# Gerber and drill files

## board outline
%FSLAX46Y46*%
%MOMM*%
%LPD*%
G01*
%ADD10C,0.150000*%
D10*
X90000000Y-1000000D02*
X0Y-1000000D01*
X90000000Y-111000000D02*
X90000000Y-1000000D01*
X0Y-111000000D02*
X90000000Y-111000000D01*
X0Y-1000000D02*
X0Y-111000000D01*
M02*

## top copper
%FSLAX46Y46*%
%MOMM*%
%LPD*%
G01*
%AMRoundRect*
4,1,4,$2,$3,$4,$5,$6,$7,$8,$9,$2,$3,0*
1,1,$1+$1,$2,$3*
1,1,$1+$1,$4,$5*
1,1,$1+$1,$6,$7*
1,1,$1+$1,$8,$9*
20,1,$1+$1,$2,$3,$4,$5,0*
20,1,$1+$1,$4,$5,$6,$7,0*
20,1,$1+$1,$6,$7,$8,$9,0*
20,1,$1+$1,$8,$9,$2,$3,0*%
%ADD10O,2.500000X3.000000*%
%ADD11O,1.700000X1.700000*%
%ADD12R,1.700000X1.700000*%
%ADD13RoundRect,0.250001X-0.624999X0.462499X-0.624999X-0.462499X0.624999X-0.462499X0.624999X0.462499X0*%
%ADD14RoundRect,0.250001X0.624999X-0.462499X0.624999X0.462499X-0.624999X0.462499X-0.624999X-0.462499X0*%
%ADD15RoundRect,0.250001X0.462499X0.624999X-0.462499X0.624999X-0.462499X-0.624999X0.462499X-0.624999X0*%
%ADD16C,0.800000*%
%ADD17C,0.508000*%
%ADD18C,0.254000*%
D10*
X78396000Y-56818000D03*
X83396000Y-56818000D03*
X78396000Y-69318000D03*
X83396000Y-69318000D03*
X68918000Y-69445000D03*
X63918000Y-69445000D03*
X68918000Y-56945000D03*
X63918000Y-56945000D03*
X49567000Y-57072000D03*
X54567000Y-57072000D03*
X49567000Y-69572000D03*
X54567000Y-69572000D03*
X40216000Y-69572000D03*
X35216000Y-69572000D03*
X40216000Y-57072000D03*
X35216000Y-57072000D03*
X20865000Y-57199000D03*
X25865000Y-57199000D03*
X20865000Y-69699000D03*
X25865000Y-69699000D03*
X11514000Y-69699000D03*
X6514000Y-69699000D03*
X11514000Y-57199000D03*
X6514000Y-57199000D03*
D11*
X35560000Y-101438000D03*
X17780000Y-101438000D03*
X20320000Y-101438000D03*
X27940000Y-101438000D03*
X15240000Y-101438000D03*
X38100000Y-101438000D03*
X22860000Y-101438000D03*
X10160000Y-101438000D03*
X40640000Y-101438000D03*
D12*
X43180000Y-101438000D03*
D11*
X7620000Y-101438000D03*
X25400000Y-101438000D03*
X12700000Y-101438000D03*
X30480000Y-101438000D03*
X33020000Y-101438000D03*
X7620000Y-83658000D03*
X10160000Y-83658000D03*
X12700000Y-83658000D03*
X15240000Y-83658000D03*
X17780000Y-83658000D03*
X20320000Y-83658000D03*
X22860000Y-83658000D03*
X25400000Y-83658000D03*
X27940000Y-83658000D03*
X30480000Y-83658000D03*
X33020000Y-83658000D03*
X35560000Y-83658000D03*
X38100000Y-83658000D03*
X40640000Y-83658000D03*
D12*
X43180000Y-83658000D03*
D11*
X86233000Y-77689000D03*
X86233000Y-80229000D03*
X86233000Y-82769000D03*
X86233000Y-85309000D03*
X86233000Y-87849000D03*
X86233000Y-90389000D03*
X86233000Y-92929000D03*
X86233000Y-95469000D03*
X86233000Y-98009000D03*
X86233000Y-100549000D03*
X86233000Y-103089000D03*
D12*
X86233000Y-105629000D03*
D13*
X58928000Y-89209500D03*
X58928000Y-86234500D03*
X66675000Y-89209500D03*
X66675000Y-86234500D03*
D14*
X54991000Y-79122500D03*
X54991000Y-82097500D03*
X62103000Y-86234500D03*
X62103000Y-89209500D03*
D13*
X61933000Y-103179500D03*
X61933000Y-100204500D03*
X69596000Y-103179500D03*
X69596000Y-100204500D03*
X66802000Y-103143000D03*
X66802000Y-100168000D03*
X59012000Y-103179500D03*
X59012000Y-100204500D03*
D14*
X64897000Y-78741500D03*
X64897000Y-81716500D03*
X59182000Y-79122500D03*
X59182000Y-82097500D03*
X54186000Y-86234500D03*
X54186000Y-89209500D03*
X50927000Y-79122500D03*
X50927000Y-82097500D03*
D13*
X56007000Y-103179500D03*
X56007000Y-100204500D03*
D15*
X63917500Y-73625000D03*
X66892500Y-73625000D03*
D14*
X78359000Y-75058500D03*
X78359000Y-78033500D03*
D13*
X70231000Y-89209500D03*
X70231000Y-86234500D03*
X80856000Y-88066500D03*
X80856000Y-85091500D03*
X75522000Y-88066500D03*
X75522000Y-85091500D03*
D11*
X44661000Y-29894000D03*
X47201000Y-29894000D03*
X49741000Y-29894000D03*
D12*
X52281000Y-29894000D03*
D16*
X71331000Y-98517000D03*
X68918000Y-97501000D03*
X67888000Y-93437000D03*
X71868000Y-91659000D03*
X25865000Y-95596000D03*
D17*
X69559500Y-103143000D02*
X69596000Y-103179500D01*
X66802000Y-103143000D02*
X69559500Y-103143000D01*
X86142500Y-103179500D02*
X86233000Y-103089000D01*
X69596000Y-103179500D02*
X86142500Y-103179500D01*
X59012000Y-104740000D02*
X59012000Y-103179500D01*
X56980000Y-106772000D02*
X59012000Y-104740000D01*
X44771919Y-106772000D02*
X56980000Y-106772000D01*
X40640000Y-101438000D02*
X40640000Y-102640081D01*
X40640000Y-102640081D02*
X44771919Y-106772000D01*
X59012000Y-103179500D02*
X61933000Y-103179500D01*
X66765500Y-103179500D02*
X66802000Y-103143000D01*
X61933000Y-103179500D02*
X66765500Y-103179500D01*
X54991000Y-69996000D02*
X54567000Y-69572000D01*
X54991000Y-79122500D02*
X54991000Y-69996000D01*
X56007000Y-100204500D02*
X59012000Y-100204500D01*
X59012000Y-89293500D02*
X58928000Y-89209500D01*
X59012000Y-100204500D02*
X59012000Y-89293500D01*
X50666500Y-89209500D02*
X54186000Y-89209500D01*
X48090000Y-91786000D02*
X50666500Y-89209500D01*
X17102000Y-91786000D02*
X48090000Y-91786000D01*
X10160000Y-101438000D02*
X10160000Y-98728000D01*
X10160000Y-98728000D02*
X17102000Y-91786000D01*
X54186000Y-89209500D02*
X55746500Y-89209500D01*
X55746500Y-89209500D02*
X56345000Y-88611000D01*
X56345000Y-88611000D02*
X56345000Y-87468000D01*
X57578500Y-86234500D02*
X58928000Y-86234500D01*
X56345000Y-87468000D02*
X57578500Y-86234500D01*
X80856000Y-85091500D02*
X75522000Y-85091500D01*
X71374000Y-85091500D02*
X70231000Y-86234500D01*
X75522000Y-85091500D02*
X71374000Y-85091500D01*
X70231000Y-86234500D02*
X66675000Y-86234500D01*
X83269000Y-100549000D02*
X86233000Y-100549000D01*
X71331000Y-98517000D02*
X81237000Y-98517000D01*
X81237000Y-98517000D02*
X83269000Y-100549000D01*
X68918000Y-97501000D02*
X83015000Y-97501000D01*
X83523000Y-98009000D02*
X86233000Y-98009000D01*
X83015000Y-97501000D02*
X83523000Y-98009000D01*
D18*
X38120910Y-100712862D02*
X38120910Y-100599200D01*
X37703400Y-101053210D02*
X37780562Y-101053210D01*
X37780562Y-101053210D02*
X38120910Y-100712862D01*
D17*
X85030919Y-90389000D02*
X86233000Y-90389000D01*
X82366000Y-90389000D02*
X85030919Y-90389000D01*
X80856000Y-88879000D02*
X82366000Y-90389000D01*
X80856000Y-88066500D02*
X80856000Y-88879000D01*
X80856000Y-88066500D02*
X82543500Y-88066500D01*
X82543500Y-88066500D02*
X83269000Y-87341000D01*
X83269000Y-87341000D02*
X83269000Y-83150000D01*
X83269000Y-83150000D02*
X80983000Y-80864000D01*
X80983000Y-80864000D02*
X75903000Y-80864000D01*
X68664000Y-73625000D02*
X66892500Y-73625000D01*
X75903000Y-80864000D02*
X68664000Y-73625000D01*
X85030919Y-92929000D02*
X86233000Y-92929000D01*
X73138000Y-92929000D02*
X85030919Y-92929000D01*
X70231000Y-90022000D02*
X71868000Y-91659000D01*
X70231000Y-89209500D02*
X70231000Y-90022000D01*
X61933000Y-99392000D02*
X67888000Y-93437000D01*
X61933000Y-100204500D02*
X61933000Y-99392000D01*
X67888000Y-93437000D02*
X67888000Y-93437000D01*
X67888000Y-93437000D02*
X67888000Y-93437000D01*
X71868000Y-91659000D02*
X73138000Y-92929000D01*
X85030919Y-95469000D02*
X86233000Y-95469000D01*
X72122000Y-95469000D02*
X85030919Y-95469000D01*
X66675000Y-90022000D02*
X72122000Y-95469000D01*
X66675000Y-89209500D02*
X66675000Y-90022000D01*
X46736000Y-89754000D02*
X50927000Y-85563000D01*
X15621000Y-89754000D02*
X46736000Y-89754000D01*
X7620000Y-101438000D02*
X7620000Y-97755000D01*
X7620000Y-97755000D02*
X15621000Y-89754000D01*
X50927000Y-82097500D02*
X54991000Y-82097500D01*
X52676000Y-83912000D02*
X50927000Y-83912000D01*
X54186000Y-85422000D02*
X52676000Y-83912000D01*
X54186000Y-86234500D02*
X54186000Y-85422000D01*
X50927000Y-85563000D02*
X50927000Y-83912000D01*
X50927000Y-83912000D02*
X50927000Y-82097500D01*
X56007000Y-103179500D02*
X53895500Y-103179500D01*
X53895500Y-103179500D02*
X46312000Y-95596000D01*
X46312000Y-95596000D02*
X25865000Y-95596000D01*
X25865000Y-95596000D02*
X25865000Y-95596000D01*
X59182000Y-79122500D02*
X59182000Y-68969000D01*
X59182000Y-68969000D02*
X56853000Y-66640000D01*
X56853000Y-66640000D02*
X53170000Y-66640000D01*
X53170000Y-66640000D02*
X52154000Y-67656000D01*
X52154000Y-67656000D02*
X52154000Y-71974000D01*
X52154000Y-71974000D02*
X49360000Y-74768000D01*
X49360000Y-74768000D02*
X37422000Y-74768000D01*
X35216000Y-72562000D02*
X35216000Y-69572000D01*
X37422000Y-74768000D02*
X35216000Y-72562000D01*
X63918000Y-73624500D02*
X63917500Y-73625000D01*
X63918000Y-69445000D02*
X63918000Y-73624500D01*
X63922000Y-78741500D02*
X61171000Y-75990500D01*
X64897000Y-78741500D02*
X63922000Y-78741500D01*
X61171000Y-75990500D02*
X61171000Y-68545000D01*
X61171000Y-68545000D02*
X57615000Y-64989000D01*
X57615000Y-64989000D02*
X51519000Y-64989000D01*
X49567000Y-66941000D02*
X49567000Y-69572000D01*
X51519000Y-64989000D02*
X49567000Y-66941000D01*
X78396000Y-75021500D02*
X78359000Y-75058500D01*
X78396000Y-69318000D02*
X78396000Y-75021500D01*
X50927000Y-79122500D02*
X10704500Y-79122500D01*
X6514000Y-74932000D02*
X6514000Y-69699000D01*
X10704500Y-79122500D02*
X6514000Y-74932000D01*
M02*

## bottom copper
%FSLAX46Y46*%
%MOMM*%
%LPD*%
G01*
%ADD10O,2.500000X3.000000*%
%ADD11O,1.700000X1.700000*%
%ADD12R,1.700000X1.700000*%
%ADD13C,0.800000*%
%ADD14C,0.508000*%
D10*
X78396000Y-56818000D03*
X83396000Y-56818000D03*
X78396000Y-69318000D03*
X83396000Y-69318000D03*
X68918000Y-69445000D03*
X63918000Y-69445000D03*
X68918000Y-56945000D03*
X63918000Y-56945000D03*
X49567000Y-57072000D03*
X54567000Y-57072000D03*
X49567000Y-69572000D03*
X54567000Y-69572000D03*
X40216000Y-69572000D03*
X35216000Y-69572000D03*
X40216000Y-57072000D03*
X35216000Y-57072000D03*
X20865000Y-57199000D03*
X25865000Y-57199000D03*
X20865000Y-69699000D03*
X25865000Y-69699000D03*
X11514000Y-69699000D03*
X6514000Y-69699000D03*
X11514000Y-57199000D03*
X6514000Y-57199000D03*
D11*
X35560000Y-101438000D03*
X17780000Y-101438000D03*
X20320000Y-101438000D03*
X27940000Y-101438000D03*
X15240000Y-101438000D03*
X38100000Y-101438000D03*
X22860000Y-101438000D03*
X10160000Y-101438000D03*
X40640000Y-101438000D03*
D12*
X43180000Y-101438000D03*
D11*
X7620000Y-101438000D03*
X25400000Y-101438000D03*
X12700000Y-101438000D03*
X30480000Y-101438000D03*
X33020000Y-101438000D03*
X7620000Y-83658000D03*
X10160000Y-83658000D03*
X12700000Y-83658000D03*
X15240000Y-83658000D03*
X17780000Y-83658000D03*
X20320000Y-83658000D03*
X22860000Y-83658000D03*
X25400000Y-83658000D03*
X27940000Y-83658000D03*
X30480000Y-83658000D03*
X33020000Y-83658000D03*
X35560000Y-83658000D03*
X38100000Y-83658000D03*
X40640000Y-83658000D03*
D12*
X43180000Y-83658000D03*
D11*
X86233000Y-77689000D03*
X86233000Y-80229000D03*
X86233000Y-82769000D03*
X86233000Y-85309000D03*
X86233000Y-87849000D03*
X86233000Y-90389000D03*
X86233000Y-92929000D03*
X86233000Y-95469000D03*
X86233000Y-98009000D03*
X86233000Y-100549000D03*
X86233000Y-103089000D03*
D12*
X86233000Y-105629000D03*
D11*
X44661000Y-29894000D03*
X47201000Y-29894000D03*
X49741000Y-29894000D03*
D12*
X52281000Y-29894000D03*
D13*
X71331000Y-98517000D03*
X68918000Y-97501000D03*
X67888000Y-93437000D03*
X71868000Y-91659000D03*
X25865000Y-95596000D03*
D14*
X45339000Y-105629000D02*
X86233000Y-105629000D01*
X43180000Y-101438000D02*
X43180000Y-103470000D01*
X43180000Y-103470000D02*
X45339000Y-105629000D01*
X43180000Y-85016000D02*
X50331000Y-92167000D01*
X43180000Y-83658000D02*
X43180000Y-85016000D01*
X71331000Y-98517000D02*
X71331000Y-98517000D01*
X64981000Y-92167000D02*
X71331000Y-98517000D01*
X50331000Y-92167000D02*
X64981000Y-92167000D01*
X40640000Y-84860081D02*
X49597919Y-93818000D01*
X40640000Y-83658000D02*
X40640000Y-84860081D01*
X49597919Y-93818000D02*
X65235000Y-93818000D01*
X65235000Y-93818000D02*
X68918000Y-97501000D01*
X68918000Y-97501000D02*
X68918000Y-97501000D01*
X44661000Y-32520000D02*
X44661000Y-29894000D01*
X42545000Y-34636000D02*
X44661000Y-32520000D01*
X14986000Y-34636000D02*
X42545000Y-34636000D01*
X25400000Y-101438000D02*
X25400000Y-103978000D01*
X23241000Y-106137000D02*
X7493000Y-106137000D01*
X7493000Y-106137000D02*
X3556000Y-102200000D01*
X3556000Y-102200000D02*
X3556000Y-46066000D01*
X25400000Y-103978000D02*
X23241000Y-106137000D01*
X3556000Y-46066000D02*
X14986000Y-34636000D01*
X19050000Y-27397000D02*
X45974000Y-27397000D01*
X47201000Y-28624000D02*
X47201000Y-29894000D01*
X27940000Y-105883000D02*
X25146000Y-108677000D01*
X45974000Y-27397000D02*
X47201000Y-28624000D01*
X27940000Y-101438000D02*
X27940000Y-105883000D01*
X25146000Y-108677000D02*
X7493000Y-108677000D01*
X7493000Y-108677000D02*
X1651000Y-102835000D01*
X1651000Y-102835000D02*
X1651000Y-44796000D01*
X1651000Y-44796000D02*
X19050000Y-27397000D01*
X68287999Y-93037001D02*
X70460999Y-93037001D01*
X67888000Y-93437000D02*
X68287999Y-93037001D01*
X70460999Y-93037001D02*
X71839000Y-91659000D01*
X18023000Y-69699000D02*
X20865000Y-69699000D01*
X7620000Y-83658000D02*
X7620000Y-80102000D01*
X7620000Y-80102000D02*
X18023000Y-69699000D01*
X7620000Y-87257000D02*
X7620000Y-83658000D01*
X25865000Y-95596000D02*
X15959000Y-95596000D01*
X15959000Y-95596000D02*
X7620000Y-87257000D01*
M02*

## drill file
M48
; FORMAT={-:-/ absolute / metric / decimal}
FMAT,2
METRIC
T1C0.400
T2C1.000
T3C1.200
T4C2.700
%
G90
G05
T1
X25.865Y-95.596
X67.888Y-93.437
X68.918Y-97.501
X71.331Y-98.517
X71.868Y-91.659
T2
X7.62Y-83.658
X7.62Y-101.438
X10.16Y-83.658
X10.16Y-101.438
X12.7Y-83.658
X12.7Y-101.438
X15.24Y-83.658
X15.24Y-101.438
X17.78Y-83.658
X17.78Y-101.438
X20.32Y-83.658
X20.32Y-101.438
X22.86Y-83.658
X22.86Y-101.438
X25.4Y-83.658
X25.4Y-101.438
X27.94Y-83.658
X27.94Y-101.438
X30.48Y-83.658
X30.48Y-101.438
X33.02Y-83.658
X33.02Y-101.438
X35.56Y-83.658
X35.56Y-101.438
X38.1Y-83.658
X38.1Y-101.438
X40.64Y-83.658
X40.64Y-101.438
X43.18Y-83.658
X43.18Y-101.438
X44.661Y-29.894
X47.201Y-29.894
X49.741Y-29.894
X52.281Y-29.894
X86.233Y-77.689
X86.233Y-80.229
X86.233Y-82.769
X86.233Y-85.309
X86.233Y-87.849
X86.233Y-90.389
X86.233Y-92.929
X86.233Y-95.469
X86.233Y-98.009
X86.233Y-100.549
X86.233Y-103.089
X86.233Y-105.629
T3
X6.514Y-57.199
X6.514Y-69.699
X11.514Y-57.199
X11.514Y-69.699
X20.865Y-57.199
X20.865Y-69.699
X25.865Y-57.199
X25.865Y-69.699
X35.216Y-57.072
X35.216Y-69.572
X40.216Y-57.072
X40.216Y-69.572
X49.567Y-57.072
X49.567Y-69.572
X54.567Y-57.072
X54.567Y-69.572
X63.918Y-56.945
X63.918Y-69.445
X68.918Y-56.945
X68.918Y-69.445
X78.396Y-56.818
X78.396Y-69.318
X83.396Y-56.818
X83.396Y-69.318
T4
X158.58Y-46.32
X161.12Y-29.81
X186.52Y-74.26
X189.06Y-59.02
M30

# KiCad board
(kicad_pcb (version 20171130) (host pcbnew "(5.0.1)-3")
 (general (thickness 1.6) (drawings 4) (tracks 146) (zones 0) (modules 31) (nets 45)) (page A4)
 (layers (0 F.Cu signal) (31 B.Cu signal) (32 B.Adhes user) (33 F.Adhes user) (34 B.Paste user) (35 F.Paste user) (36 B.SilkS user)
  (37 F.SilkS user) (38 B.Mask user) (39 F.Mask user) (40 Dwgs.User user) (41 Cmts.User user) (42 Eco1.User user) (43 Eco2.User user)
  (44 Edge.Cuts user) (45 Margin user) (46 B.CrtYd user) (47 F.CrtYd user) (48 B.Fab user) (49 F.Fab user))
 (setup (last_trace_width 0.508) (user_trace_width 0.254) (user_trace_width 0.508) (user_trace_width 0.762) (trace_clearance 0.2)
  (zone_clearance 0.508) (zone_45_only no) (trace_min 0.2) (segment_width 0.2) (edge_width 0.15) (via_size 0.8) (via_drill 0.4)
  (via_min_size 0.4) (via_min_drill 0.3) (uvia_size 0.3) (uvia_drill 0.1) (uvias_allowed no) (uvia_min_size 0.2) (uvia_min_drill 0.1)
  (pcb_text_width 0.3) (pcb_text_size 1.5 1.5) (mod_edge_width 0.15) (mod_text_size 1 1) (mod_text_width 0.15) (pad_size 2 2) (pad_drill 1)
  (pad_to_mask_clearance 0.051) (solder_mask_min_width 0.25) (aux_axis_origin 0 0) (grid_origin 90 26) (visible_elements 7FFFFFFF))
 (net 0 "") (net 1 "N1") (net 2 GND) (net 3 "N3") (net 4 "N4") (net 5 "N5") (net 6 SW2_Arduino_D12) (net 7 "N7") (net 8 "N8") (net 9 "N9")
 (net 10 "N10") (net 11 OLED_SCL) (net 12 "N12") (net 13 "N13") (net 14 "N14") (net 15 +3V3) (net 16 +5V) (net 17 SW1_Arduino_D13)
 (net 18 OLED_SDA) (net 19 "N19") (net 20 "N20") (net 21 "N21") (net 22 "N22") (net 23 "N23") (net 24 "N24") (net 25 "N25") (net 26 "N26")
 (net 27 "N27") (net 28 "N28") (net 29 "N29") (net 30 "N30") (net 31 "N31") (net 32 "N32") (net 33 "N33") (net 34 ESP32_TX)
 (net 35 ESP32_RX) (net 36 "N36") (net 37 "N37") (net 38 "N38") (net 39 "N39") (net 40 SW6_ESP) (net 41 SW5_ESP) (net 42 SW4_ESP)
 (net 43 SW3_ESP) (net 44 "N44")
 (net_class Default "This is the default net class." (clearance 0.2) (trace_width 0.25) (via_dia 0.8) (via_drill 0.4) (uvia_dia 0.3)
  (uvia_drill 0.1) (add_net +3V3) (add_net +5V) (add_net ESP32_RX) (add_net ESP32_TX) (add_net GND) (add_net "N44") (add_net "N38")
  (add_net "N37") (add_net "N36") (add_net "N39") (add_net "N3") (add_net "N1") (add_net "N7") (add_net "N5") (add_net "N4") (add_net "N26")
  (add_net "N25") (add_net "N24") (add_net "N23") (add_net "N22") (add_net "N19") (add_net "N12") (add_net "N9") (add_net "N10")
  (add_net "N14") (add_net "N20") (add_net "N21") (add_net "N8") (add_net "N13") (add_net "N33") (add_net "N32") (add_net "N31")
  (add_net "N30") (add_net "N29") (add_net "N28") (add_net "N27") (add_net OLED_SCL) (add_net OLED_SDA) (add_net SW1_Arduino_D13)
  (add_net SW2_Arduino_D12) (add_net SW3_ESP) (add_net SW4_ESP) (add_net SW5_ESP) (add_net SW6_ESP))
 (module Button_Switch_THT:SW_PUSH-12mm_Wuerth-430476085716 (layer F.Cu) (at 83.396 56.818 270)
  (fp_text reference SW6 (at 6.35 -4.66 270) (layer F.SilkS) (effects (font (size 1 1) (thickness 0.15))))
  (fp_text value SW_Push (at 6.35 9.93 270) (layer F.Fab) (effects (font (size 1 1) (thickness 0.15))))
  (pad 2 thru_hole oval (at 0 5 270) (size 3 2.5) (drill 1.2) (layers *.Cu *.Mask) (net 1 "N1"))
  (pad 1 thru_hole oval (at 0 0 270) (size 3 2.5) (drill 1.2) (layers *.Cu *.Mask) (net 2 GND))
  (pad 2 thru_hole oval (at 12.5 5 270) (size 3 2.5) (drill 1.2) (layers *.Cu *.Mask) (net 1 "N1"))
  (pad 1 thru_hole oval (at 12.5 0 270) (size 3 2.5) (drill 1.2) (layers *.Cu *.Mask) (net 2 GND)))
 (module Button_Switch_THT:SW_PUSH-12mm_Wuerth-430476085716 (layer F.Cu) (at 68.918 56.945 270)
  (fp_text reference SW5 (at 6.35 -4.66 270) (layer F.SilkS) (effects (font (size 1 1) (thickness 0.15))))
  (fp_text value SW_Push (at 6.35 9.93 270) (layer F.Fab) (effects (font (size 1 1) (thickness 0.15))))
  (pad 1 thru_hole oval (at 12.5 0 270) (size 3 2.5) (drill 1.2) (layers *.Cu *.Mask) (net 2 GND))
  (pad 2 thru_hole oval (at 12.5 5 270) (size 3 2.5) (drill 1.2) (layers *.Cu *.Mask) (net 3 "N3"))
  (pad 1 thru_hole oval (at 0 0 270) (size 3 2.5) (drill 1.2) (layers *.Cu *.Mask) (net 2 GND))
  (pad 2 thru_hole oval (at 0 5 270) (size 3 2.5) (drill 1.2) (layers *.Cu *.Mask) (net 3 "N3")))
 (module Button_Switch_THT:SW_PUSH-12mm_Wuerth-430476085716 (layer F.Cu) (at 54.567 57.072 270)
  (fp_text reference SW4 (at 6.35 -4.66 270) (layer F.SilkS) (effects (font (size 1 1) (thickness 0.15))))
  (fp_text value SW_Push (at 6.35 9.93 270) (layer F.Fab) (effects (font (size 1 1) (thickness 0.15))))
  (pad 2 thru_hole oval (at 0 5 270) (size 3 2.5) (drill 1.2) (layers *.Cu *.Mask) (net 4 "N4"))
  (pad 1 thru_hole oval (at 0 0 270) (size 3 2.5) (drill 1.2) (layers *.Cu *.Mask) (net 2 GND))
  (pad 2 thru_hole oval (at 12.5 5 270) (size 3 2.5) (drill 1.2) (layers *.Cu *.Mask) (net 4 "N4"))
  (pad 1 thru_hole oval (at 12.5 0 270) (size 3 2.5) (drill 1.2) (layers *.Cu *.Mask) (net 2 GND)))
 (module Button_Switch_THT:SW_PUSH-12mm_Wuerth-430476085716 (layer F.Cu) (at 40.216 57.072 270)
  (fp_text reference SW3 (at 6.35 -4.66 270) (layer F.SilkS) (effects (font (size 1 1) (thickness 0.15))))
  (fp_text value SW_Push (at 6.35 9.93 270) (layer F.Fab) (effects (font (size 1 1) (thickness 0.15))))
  (pad 1 thru_hole oval (at 12.5 0 270) (size 3 2.5) (drill 1.2) (layers *.Cu *.Mask) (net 2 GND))
  (pad 2 thru_hole oval (at 12.5 5 270) (size 3 2.5) (drill 1.2) (layers *.Cu *.Mask) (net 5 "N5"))
  (pad 1 thru_hole oval (at 0 0 270) (size 3 2.5) (drill 1.2) (layers *.Cu *.Mask) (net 2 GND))
  (pad 2 thru_hole oval (at 0 5 270) (size 3 2.5) (drill 1.2) (layers *.Cu *.Mask) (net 5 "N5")))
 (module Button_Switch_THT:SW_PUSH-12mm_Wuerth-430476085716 (layer F.Cu) (at 25.865 57.199 270)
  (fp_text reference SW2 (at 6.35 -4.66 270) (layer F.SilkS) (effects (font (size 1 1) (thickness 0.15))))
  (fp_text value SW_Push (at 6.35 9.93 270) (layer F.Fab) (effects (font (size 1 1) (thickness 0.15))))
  (pad 2 thru_hole oval (at 0 5 270) (size 3 2.5) (drill 1.2) (layers *.Cu *.Mask) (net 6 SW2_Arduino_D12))
  (pad 1 thru_hole oval (at 0 0 270) (size 3 2.5) (drill 1.2) (layers *.Cu *.Mask) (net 2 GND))
  (pad 2 thru_hole oval (at 12.5 5 270) (size 3 2.5) (drill 1.2) (layers *.Cu *.Mask) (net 6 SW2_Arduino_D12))
  (pad 1 thru_hole oval (at 12.5 0 270) (size 3 2.5) (drill 1.2) (layers *.Cu *.Mask) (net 2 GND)))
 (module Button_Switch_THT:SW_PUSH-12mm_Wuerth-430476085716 (layer F.Cu) (at 11.514 57.199 270)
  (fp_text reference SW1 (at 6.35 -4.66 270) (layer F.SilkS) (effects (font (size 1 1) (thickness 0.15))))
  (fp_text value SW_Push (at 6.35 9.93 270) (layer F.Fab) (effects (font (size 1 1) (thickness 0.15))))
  (pad 1 thru_hole oval (at 12.5 0 270) (size 3 2.5) (drill 1.2) (layers *.Cu *.Mask) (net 2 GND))
  (pad 2 thru_hole oval (at 12.5 5 270) (size 3 2.5) (drill 1.2) (layers *.Cu *.Mask) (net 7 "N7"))
  (pad 1 thru_hole oval (at 0 0 270) (size 3 2.5) (drill 1.2) (layers *.Cu *.Mask) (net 2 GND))
  (pad 2 thru_hole oval (at 0 5 270) (size 3 2.5) (drill 1.2) (layers *.Cu *.Mask) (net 7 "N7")))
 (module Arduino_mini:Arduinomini (layer F.Cu) (at 43.18 91.278 270)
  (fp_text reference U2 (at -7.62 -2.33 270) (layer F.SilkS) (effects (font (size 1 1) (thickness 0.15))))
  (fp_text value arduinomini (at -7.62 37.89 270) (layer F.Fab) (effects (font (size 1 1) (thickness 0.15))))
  (pad 27 thru_hole oval (at 10.16 7.62 270) (size 1.7 1.7) (drill 1) (layers *.Cu *.Mask) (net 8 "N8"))
  (pad 20 thru_hole oval (at 10.16 25.4 270) (size 1.7 1.7) (drill 1) (layers *.Cu *.Mask) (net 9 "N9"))
  (pad 21 thru_hole oval (at 10.16 22.86 270) (size 1.7 1.7) (drill 1) (layers *.Cu *.Mask) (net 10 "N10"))
  (pad 24 thru_hole oval (at 10.16 15.24 270) (size 1.7 1.7) (drill 1) (layers *.Cu *.Mask) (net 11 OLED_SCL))
  (pad 19 thru_hole oval (at 10.16 27.94 270) (size 1.7 1.7) (drill 1) (layers *.Cu *.Mask) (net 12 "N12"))
  (pad 28 thru_hole oval (at 10.16 5.08 270) (size 1.7 1.7) (drill 1) (layers *.Cu *.Mask) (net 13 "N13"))
  (pad 22 thru_hole oval (at 10.16 20.32 270) (size 1.7 1.7) (drill 1) (layers *.Cu *.Mask) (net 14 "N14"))
  (pad 17 thru_hole oval (at 10.16 33.02 270) (size 1.7 1.7) (drill 1) (layers *.Cu *.Mask) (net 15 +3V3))
  (pad 29 thru_hole oval (at 10.16 2.54 270) (size 1.7 1.7) (drill 1) (layers *.Cu *.Mask) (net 2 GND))
  (pad 30 thru_hole rect (at 10.16 0 270) (size 1.7 1.7) (drill 1) (layers *.Cu *.Mask) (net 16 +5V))
  (pad 16 thru_hole oval (at 10.16 35.56 270) (size 1.7 1.7) (drill 1) (layers *.Cu *.Mask) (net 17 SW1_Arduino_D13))
  (pad 23 thru_hole oval (at 10.16 17.78 270) (size 1.7 1.7) (drill 1) (layers *.Cu *.Mask) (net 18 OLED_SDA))
  (pad 18 thru_hole oval (at 10.16 30.48 270) (size 1.7 1.7) (drill 1) (layers *.Cu *.Mask) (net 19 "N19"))
  (pad 25 thru_hole oval (at 10.16 12.7 270) (size 1.7 1.7) (drill 1) (layers *.Cu *.Mask) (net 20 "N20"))
  (pad 26 thru_hole oval (at 10.16 10.16 270) (size 1.7 1.7) (drill 1) (layers *.Cu *.Mask) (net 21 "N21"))
  (pad 15 thru_hole oval (at -7.62 35.56 270) (size 1.7 1.7) (drill 1) (layers *.Cu *.Mask) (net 6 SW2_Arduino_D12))
  (pad 14 thru_hole oval (at -7.62 33.02 270) (size 1.7 1.7) (drill 1) (layers *.Cu *.Mask) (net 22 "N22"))
  (pad 13 thru_hole oval (at -7.62 30.48 270) (size 1.7 1.7) (drill 1) (layers *.Cu *.Mask) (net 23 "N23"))
  (pad 12 thru_hole oval (at -7.62 27.94 270) (size 1.7 1.7) (drill 1) (layers *.Cu *.Mask) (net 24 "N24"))
  (pad 11 thru_hole oval (at -7.62 25.4 270) (size 1.7 1.7) (drill 1) (layers *.Cu *.Mask) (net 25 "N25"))
  (pad 10 thru_hole oval (at -7.62 22.86 270) (size 1.7 1.7) (drill 1) (layers *.Cu *.Mask) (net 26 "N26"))
  (pad 9 thru_hole oval (at -7.62 20.32 270) (size 1.7 1.7) (drill 1) (layers *.Cu *.Mask) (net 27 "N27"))
  (pad 8 thru_hole oval (at -7.62 17.78 270) (size 1.7 1.7) (drill 1) (layers *.Cu *.Mask) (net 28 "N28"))
  (pad 7 thru_hole oval (at -7.62 15.24 270) (size 1.7 1.7) (drill 1) (layers *.Cu *.Mask) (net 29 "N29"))
  (pad 6 thru_hole oval (at -7.62 12.7 270) (size 1.7 1.7) (drill 1) (layers *.Cu *.Mask) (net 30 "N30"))
  (pad 5 thru_hole oval (at -7.62 10.16 270) (size 1.7 1.7) (drill 1) (layers *.Cu *.Mask) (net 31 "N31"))
  (pad 4 thru_hole oval (at -7.62 7.62 270) (size 1.7 1.7) (drill 1) (layers *.Cu *.Mask) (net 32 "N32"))
  (pad 3 thru_hole oval (at -7.62 5.08 270) (size 1.7 1.7) (drill 1) (layers *.Cu *.Mask) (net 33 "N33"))
  (pad 2 thru_hole oval (at -7.62 2.54 270) (size 1.7 1.7) (drill 1) (layers *.Cu *.Mask) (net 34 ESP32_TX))
  (pad 1 thru_hole rect (at -7.62 0 270) (size 1.7 1.7) (drill 1) (layers *.Cu *.Mask) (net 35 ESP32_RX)))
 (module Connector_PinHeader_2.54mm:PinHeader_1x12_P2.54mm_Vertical (layer F.Cu) (at 86.233 105.629 180)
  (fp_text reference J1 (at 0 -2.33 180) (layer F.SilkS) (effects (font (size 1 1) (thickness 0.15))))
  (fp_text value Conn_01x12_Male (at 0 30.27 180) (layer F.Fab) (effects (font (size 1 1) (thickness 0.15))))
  (pad 12 thru_hole oval (at 0 27.94 180) (size 1.7 1.7) (drill 1) (layers *.Cu *.Mask) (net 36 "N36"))
  (pad 11 thru_hole oval (at 0 25.4 180) (size 1.7 1.7) (drill 1) (layers *.Cu *.Mask) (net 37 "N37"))
  (pad 10 thru_hole oval (at 0 22.86 180) (size 1.7 1.7) (drill 1) (layers *.Cu *.Mask) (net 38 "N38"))
  (pad 9 thru_hole oval (at 0 20.32 180) (size 1.7 1.7) (drill 1) (layers *.Cu *.Mask) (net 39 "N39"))
  (pad 8 thru_hole oval (at 0 17.78 180) (size 1.7 1.7) (drill 1) (layers *.Cu *.Mask) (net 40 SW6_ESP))
  (pad 7 thru_hole oval (at 0 15.24 180) (size 1.7 1.7) (drill 1) (layers *.Cu *.Mask) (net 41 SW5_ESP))
  (pad 6 thru_hole oval (at 0 12.7 180) (size 1.7 1.7) (drill 1) (layers *.Cu *.Mask) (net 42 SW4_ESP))
  (pad 5 thru_hole oval (at 0 10.16 180) (size 1.7 1.7) (drill 1) (layers *.Cu *.Mask) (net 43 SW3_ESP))
  (pad 4 thru_hole oval (at 0 7.62 180) (size 1.7 1.7) (drill 1) (layers *.Cu *.Mask) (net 34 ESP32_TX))
  (pad 3 thru_hole oval (at 0 5.08 180) (size 1.7 1.7) (drill 1) (layers *.Cu *.Mask) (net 35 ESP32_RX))
  (pad 2 thru_hole oval (at 0 2.54 180) (size 1.7 1.7) (drill 1) (layers *.Cu *.Mask) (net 2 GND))
  (pad 1 thru_hole rect (at 0 0 180) (size 1.7 1.7) (drill 1) (layers *.Cu *.Mask) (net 16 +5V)))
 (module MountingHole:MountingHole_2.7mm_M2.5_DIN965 (layer F.Cu) (at 186.52 74.26)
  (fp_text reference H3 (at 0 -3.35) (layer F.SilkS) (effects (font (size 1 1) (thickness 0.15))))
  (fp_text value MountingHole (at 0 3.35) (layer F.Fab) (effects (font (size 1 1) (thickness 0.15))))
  (pad 1 np_thru_hole circle (at 0 0) (size 2.7 2.7) (drill 2.7) (layers *.Cu *.Mask)))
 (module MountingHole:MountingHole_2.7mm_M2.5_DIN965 (layer F.Cu) (at 158.58 46.32)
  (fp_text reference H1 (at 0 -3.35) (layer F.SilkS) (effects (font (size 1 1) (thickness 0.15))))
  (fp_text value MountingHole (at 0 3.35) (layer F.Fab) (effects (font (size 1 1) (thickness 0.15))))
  (pad 1 np_thru_hole circle (at 0 0) (size 2.7 2.7) (drill 2.7) (layers *.Cu *.Mask)))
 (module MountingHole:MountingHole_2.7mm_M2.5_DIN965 (layer F.Cu) (at 189.06 59.02)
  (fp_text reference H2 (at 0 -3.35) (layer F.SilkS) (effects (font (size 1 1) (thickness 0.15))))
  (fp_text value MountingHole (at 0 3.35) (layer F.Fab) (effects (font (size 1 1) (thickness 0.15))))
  (pad 1 np_thru_hole circle (at 0 0) (size 2.7 2.7) (drill 2.7) (layers *.Cu *.Mask)))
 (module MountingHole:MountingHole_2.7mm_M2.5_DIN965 (layer F.Cu) (at 161.12 29.81)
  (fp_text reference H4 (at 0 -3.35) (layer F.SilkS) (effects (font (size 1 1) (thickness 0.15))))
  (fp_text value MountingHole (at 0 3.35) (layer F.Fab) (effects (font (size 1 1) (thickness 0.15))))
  (pad 1 np_thru_hole circle (at 0 0) (size 2.7 2.7) (drill 2.7) (layers *.Cu *.Mask)))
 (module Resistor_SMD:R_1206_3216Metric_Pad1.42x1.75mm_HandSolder (layer F.Cu) (at 58.928 87.722 270)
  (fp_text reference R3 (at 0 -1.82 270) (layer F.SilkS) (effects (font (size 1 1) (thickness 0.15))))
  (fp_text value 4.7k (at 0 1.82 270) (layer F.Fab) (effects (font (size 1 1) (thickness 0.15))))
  (pad 2 smd roundrect (at 1.4875 0 270) (size 1.425 1.75) (layers F.Cu F.Paste F.Mask) (roundrect_rratio 0.175439) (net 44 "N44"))
  (pad 1 smd roundrect (at -1.4875 0 270) (size 1.425 1.75) (layers F.Cu F.Paste F.Mask) (roundrect_rratio 0.175439) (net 15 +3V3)))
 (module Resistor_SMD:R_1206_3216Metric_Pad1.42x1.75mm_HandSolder (layer F.Cu) (at 66.675 87.722 270)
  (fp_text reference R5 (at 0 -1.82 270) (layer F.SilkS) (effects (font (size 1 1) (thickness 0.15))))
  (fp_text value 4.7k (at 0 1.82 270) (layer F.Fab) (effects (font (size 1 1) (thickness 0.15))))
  (pad 2 smd roundrect (at 1.4875 0 270) (size 1.425 1.75) (layers F.Cu F.Paste F.Mask) (roundrect_rratio 0.175439) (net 43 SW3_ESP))
  (pad 1 smd roundrect (at -1.4875 0 270) (size 1.425 1.75) (layers F.Cu F.Paste F.Mask) (roundrect_rratio 0.175439) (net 15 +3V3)))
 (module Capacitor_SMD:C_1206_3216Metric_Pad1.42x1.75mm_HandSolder (layer F.Cu) (at 54.991 80.61 90)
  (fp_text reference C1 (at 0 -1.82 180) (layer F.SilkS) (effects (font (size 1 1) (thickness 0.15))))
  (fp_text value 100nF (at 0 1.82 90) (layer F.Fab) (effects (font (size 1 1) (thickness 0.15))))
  (pad 2 smd roundrect (at 1.4875 0 90) (size 1.425 1.75) (layers F.Cu F.Paste F.Mask) (roundrect_rratio 0.175439) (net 2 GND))
  (pad 1 smd roundrect (at -1.4875 0 90) (size 1.425 1.75) (layers F.Cu F.Paste F.Mask) (roundrect_rratio 0.175439) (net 17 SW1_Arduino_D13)))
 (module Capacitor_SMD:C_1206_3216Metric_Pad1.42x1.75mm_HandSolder (layer F.Cu) (at 62.103 87.722 90)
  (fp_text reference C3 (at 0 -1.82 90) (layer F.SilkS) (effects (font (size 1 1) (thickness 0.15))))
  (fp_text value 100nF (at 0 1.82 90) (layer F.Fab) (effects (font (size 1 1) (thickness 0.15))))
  (pad 2 smd roundrect (at 1.4875 0 90) (size 1.425 1.75) (layers F.Cu F.Paste F.Mask) (roundrect_rratio 0.175439) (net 2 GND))
  (pad 1 smd roundrect (at -1.4875 0 90) (size 1.425 1.75) (layers F.Cu F.Paste F.Mask) (roundrect_rratio 0.175439) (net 43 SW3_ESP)))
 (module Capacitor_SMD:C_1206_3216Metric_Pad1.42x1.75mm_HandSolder (layer F.Cu) (at 61.933 101.692 270)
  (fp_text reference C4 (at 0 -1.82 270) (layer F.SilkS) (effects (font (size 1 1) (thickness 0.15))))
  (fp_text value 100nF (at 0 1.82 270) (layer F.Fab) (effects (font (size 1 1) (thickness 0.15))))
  (pad 2 smd roundrect (at 1.4875 0 270) (size 1.425 1.75) (layers F.Cu F.Paste F.Mask) (roundrect_rratio 0.175439) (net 2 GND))
  (pad 1 smd roundrect (at -1.4875 0 270) (size 1.425 1.75) (layers F.Cu F.Paste F.Mask) (roundrect_rratio 0.175439) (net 42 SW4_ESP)))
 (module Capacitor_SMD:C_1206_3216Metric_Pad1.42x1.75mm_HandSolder (layer F.Cu) (at 69.596 101.692 270)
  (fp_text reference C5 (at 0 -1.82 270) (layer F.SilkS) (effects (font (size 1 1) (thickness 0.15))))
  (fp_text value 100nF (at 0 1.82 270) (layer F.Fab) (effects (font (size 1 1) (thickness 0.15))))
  (pad 2 smd roundrect (at 1.4875 0 270) (size 1.425 1.75) (layers F.Cu F.Paste F.Mask) (roundrect_rratio 0.175439) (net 2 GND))
  (pad 1 smd roundrect (at -1.4875 0 270) (size 1.425 1.75) (layers F.Cu F.Paste F.Mask) (roundrect_rratio 0.175439) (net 41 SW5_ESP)))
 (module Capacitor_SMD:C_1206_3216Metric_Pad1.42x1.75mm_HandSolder (layer F.Cu) (at 66.802 101.6555 270)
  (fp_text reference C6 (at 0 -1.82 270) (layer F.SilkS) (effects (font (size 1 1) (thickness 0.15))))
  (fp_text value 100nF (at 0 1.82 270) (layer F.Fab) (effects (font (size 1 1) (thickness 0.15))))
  (pad 2 smd roundrect (at 1.4875 0 270) (size 1.425 1.75) (layers F.Cu F.Paste F.Mask) (roundrect_rratio 0.175439) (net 2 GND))
  (pad 1 smd roundrect (at -1.4875 0 270) (size 1.425 1.75) (layers F.Cu F.Paste F.Mask) (roundrect_rratio 0.175439) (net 40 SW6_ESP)))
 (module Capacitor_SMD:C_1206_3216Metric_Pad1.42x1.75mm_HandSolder (layer F.Cu) (at 59.012 101.692 270)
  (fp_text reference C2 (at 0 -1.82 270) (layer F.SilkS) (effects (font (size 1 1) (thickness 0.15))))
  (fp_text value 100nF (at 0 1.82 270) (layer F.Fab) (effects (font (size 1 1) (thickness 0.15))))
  (pad 2 smd roundrect (at 1.4875 0 270) (size 1.425 1.75) (layers F.Cu F.Paste F.Mask) (roundrect_rratio 0.175439) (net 2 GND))
  (pad 1 smd roundrect (at -1.4875 0 270) (size 1.425 1.75) (layers F.Cu F.Paste F.Mask) (roundrect_rratio 0.175439) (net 44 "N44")))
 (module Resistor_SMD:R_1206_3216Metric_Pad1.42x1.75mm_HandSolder (layer F.Cu) (at 64.897 80.229 90)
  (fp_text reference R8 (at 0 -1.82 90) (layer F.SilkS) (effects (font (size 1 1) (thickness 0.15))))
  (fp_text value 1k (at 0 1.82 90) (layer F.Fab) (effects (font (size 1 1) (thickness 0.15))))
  (pad 2 smd roundrect (at 1.4875 0 90) (size 1.425 1.75) (layers F.Cu F.Paste F.Mask) (roundrect_rratio 0.175439) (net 4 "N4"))
  (pad 1 smd roundrect (at -1.4875 0 90) (size 1.425 1.75) (layers F.Cu F.Paste F.Mask) (roundrect_rratio 0.175439) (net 42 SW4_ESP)))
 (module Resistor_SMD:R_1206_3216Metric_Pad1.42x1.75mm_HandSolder (layer F.Cu) (at 59.182 80.61 90)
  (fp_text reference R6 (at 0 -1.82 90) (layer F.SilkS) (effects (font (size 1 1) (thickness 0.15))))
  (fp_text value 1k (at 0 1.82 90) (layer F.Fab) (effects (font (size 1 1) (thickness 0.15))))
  (pad 2 smd roundrect (at 1.4875 0 90) (size 1.425 1.75) (layers F.Cu F.Paste F.Mask) (roundrect_rratio 0.175439) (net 5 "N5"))
  (pad 1 smd roundrect (at -1.4875 0 90) (size 1.425 1.75) (layers F.Cu F.Paste F.Mask) (roundrect_rratio 0.175439) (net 43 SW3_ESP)))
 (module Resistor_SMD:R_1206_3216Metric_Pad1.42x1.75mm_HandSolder (layer F.Cu) (at 54.186 87.722 90)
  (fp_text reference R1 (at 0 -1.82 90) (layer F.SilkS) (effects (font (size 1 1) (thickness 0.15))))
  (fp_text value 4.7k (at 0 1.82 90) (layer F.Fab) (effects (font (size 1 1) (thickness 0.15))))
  (pad 2 smd roundrect (at 1.4875 0 90) (size 1.425 1.75) (layers F.Cu F.Paste F.Mask) (roundrect_rratio 0.175439) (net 17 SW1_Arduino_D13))
  (pad 1 smd roundrect (at -1.4875 0 90) (size 1.425 1.75) (layers F.Cu F.Paste F.Mask) (roundrect_rratio 0.175439) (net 15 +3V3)))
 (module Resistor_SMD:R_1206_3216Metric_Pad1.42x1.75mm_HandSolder (layer F.Cu) (at 50.927 80.61 90)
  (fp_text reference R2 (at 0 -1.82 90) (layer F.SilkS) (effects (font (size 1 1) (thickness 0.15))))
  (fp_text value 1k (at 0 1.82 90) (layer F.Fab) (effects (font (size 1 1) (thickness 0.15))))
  (pad 2 smd roundrect (at 1.4875 0 90) (size 1.425 1.75) (layers F.Cu F.Paste F.Mask) (roundrect_rratio 0.175439) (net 7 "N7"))
  (pad 1 smd roundrect (at -1.4875 0 90) (size 1.425 1.75) (layers F.Cu F.Paste F.Mask) (roundrect_rratio 0.175439) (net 17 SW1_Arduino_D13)))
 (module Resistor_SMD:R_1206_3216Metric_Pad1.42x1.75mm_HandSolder (layer F.Cu) (at 56.007 101.692 270)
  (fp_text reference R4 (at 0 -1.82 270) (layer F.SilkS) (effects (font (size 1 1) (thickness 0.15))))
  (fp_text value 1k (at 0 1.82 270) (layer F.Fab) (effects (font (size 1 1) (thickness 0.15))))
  (pad 2 smd roundrect (at 1.4875 0 270) (size 1.425 1.75) (layers F.Cu F.Paste F.Mask) (roundrect_rratio 0.175439) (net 6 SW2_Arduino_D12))
  (pad 1 smd roundrect (at -1.4875 0 270) (size 1.425 1.75) (layers F.Cu F.Paste F.Mask) (roundrect_rratio 0.175439) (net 44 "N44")))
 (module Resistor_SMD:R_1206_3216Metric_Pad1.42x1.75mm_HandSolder (layer F.Cu) (at 65.405 73.625 180)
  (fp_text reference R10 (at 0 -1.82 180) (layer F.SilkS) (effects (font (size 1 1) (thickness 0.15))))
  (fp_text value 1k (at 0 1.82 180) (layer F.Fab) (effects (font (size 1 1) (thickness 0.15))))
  (pad 2 smd roundrect (at 1.4875 0 180) (size 1.425 1.75) (layers F.Cu F.Paste F.Mask) (roundrect_rratio 0.175439) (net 3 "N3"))
  (pad 1 smd roundrect (at -1.4875 0 180) (size 1.425 1.75) (layers F.Cu F.Paste F.Mask) (roundrect_rratio 0.175439) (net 41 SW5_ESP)))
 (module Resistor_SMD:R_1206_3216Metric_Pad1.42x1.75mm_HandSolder (layer F.Cu) (at 78.359 76.546 90)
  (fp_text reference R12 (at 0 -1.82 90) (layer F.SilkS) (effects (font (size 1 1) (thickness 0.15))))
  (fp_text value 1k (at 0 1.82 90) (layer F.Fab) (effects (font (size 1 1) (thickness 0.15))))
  (pad 2 smd roundrect (at 1.4875 0 90) (size 1.425 1.75) (layers F.Cu F.Paste F.Mask) (roundrect_rratio 0.175439) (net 1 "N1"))
  (pad 1 smd roundrect (at -1.4875 0 90) (size 1.425 1.75) (layers F.Cu F.Paste F.Mask) (roundrect_rratio 0.175439) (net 40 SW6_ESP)))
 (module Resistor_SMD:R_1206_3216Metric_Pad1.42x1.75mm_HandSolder (layer F.Cu) (at 70.231 87.722 270)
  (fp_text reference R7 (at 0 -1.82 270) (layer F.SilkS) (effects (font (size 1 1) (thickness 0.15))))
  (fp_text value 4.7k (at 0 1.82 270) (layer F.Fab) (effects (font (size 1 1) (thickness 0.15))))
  (pad 2 smd roundrect (at 1.4875 0 270) (size 1.425 1.75) (layers F.Cu F.Paste F.Mask) (roundrect_rratio 0.175439) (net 42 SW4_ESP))
  (pad 1 smd roundrect (at -1.4875 0 270) (size 1.425 1.75) (layers F.Cu F.Paste F.Mask) (roundrect_rratio 0.175439) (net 15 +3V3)))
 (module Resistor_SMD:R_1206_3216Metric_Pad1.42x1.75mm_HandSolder (layer F.Cu) (at 80.856 86.579 270)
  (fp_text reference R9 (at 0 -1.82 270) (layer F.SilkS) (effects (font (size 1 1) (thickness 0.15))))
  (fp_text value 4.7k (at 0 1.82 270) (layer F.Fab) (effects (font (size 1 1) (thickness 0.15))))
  (pad 2 smd roundrect (at 1.4875 0 270) (size 1.425 1.75) (layers F.Cu F.Paste F.Mask) (roundrect_rratio 0.175439) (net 41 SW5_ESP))
  (pad 1 smd roundrect (at -1.4875 0 270) (size 1.425 1.75) (layers F.Cu F.Paste F.Mask) (roundrect_rratio 0.175439) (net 15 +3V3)))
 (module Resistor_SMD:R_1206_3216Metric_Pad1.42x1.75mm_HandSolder (layer F.Cu) (at 75.522 86.579 270)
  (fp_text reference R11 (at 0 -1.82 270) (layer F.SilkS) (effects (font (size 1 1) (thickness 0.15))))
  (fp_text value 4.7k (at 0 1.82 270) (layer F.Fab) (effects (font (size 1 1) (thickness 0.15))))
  (pad 2 smd roundrect (at 1.4875 0 270) (size 1.425 1.75) (layers F.Cu F.Paste F.Mask) (roundrect_rratio 0.175439) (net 40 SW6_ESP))
  (pad 1 smd roundrect (at -1.4875 0 270) (size 1.425 1.75) (layers F.Cu F.Paste F.Mask) (roundrect_rratio 0.175439) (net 15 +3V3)))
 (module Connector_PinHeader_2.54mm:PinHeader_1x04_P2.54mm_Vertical (layer F.Cu) (at 52.281 29.894 270)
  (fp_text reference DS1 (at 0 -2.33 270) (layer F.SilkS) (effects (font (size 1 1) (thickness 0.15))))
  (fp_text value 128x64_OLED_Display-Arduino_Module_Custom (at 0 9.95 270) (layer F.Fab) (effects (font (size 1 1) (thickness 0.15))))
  (pad 4 thru_hole oval (at 0 7.62 270) (size 1.7 1.7) (drill 1) (layers *.Cu *.Mask) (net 18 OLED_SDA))
  (pad 3 thru_hole oval (at 0 5.08 270) (size 1.7 1.7) (drill 1) (layers *.Cu *.Mask) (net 11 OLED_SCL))
  (pad 2 thru_hole oval (at 0 2.54 270) (size 1.7 1.7) (drill 1) (layers *.Cu *.Mask) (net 2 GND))
  (pad 1 thru_hole rect (at 0 0 270) (size 1.7 1.7) (drill 1) (layers *.Cu *.Mask) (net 15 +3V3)))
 (gr_line (start 90 1) (end 0 1) (layer Edge.Cuts) (width 0.15))
 (gr_line (start 90 111) (end 90 1) (layer Edge.Cuts) (width 0.15))
 (gr_line (start 0 111) (end 90 111) (layer Edge.Cuts) (width 0.15))
 (gr_line (start 0 1) (end 0 111) (layer Edge.Cuts) (width 0.15))
 (segment (start 69.5595 103.143) (end 69.596 103.1795) (width 0.508) (layer F.Cu) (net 2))
 (segment (start 66.802 103.143) (end 69.5595 103.143) (width 0.508) (layer F.Cu) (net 2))
 (segment (start 86.1425 103.1795) (end 86.233 103.089) (width 0.508) (layer F.Cu) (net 2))
 (segment (start 69.596 103.1795) (end 86.1425 103.1795) (width 0.508) (layer F.Cu) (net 2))
 (segment (start 59.012 104.74) (end 59.012 103.1795) (width 0.508) (layer F.Cu) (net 2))
 (segment (start 56.98 106.772) (end 59.012 104.74) (width 0.508) (layer F.Cu) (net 2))
 (segment (start 44.771919 106.772) (end 56.98 106.772) (width 0.508) (layer F.Cu) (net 2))
 (segment (start 40.64 101.438) (end 40.64 102.640081) (width 0.508) (layer F.Cu) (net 2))
 (segment (start 40.64 102.640081) (end 44.771919 106.772) (width 0.508) (layer F.Cu) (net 2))
 (segment (start 59.012 103.1795) (end 61.933 103.1795) (width 0.508) (layer F.Cu) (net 2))
 (segment (start 66.7655 103.1795) (end 66.802 103.143) (width 0.508) (layer F.Cu) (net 2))
 (segment (start 61.933 103.1795) (end 66.7655 103.1795) (width 0.508) (layer F.Cu) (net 2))
 (segment (start 54.991 69.996) (end 54.567 69.572) (width 0.508) (layer F.Cu) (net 2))
 (segment (start 54.991 79.1225) (end 54.991 69.996) (width 0.508) (layer F.Cu) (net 2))
 (segment (start 56.007 100.2045) (end 59.012 100.2045) (width 0.508) (layer F.Cu) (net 44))
 (segment (start 59.012 89.2935) (end 58.928 89.2095) (width 0.508) (layer F.Cu) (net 44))
 (segment (start 59.012 100.2045) (end 59.012 89.2935) (width 0.508) (layer F.Cu) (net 44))
 (segment (start 50.6665 89.2095) (end 54.186 89.2095) (width 0.508) (layer F.Cu) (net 15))
 (segment (start 48.09 91.786) (end 50.6665 89.2095) (width 0.508) (layer F.Cu) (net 15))
 (segment (start 17.102 91.786) (end 48.09 91.786) (width 0.508) (layer F.Cu) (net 15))
 (segment (start 10.16 101.438) (end 10.16 98.728) (width 0.508) (layer F.Cu) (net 15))
 (segment (start 10.16 98.728) (end 17.102 91.786) (width 0.508) (layer F.Cu) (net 15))
 (segment (start 54.186 89.2095) (end 55.7465 89.2095) (width 0.508) (layer F.Cu) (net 15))
 (segment (start 55.7465 89.2095) (end 56.345 88.611) (width 0.508) (layer F.Cu) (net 15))
 (segment (start 56.345 88.611) (end 56.345 87.468) (width 0.508) (layer F.Cu) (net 15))
 (segment (start 57.5785 86.2345) (end 58.928 86.2345) (width 0.508) (layer F.Cu) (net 15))
 (segment (start 56.345 87.468) (end 57.5785 86.2345) (width 0.508) (layer F.Cu) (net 15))
 (segment (start 80.856 85.0915) (end 75.522 85.0915) (width 0.508) (layer F.Cu) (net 15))
 (segment (start 71.374 85.0915) (end 70.231 86.2345) (width 0.508) (layer F.Cu) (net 15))
 (segment (start 75.522 85.0915) (end 71.374 85.0915) (width 0.508) (layer F.Cu) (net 15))
 (segment (start 70.231 86.2345) (end 66.675 86.2345) (width 0.508) (layer F.Cu) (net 15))
 (segment (start 45.339 105.629) (end 86.233 105.629) (width 0.508) (layer B.Cu) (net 16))
 (segment (start 43.18 101.438) (end 43.18 103.47) (width 0.508) (layer B.Cu) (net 16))
 (segment (start 43.18 103.47) (end 45.339 105.629) (width 0.508) (layer B.Cu) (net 16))
 (segment (start 43.18 85.016) (end 50.331 92.167) (width 0.508) (layer B.Cu) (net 35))
 (segment (start 43.18 83.658) (end 43.18 85.016) (width 0.508) (layer B.Cu) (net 35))
 (segment (start 71.331 98.517) (end 71.331 98.517) (width 0.508) (layer B.Cu) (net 35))
 (via (at 71.331 98.517) (size 0.8) (drill 0.4) (layers F.Cu B.Cu) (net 35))
 (segment (start 83.269 100.549) (end 86.233 100.549) (width 0.508) (layer F.Cu) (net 35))
 (segment (start 71.331 98.517) (end 81.237 98.517) (width 0.508) (layer F.Cu) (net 35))
 (segment (start 81.237 98.517) (end 83.269 100.549) (width 0.508) (layer F.Cu) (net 35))
 (segment (start 64.981 92.167) (end 71.331 98.517) (width 0.508) (layer B.Cu) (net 35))
 (segment (start 50.331 92.167) (end 64.981 92.167) (width 0.508) (layer B.Cu) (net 35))
 (segment (start 40.64 84.860081) (end 49.597919 93.818) (width 0.508) (layer B.Cu) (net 34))
 (segment (start 40.64 83.658) (end 40.64 84.860081) (width 0.508) (layer B.Cu) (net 34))
 (segment (start 49.597919 93.818) (end 65.235 93.818) (width 0.508) (layer B.Cu) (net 34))
 (segment (start 65.235 93.818) (end 68.918 97.501) (width 0.508) (layer B.Cu) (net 34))
 (segment (start 68.918 97.501) (end 68.918 97.501) (width 0.508) (layer B.Cu) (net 34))
 (via (at 68.918 97.501) (size 0.8) (drill 0.4) (layers F.Cu B.Cu) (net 34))
 (segment (start 68.918 97.501) (end 83.015 97.501) (width 0.508) (layer F.Cu) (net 34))
 (segment (start 83.523 98.009) (end 86.233 98.009) (width 0.508) (layer F.Cu) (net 34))
 (segment (start 83.015 97.501) (end 83.523 98.009) (width 0.508) (layer F.Cu) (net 34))
 (segment (start 38.12091 100.712862) (end 38.12091 100.5992) (width 0.254) (layer F.Cu) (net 13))
 (segment (start 37.7034 101.05321) (end 37.780562 101.05321) (width 0.254) (layer F.Cu) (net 13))
 (segment (start 37.780562 101.05321) (end 38.12091 100.712862) (width 0.254) (layer F.Cu) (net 13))
 (segment (start 44.661 32.52) (end 44.661 29.894) (width 0.508) (layer B.Cu) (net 18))
 (segment (start 42.545 34.636) (end 44.661 32.52) (width 0.508) (layer B.Cu) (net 18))
 (segment (start 14.986 34.636) (end 42.545 34.636) (width 0.508) (layer B.Cu) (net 18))
 (segment (start 25.4 101.438) (end 25.4 103.978) (width 0.508) (layer B.Cu) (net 18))
 (segment (start 23.241 106.137) (end 7.493 106.137) (width 0.508) (layer B.Cu) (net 18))
 (segment (start 7.493 106.137) (end 3.556 102.2) (width 0.508) (layer B.Cu) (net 18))
 (segment (start 3.556 102.2) (end 3.556 46.066) (width 0.508) (layer B.Cu) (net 18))
 (segment (start 25.4 103.978) (end 23.241 106.137) (width 0.508) (layer B.Cu) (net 18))
 (segment (start 3.556 46.066) (end 14.986 34.636) (width 0.508) (layer B.Cu) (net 18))
 (segment (start 19.05 27.397) (end 45.974 27.397) (width 0.508) (layer B.Cu) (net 11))
 (segment (start 47.201 28.624) (end 47.201 29.894) (width 0.508) (layer B.Cu) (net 11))
 (segment (start 27.94 105.883) (end 25.146 108.677) (width 0.508) (layer B.Cu) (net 11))
 (segment (start 45.974 27.397) (end 47.201 28.624) (width 0.508) (layer B.Cu) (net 11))
 (segment (start 27.94 101.438) (end 27.94 105.883) (width 0.508) (layer B.Cu) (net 11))
 (segment (start 25.146 108.677) (end 7.493 108.677) (width 0.508) (layer B.Cu) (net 11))
 (segment (start 7.493 108.677) (end 1.651 102.835) (width 0.508) (layer B.Cu) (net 11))
 (segment (start 1.651 102.835) (end 1.651 44.796) (width 0.508) (layer B.Cu) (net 11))
 (segment (start 1.651 44.796) (end 19.05 27.397) (width 0.508) (layer B.Cu) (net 11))
 (segment (start 85.030919 90.389) (end 86.233 90.389) (width 0.508) (layer F.Cu) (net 41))
 (segment (start 82.366 90.389) (end 85.030919 90.389) (width 0.508) (layer F.Cu) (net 41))
 (segment (start 80.856 88.879) (end 82.366 90.389) (width 0.508) (layer F.Cu) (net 41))
 (segment (start 80.856 88.0665) (end 80.856 88.879) (width 0.508) (layer F.Cu) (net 41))
 (segment (start 80.856 88.0665) (end 82.5435 88.0665) (width 0.508) (layer F.Cu) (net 41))
 (segment (start 82.5435 88.0665) (end 83.269 87.341) (width 0.508) (layer F.Cu) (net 41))
 (segment (start 83.269 87.341) (end 83.269 83.15) (width 0.508) (layer F.Cu) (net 41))
 (segment (start 83.269 83.15) (end 80.983 80.864) (width 0.508) (layer F.Cu) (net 41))
 (segment (start 80.983 80.864) (end 75.903 80.864) (width 0.508) (layer F.Cu) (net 41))
 (segment (start 68.664 73.625) (end 66.8925 73.625) (width 0.508) (layer F.Cu) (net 41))
 (segment (start 75.903 80.864) (end 68.664 73.625) (width 0.508) (layer F.Cu) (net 41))
 (segment (start 85.030919 92.929) (end 86.233 92.929) (width 0.508) (layer F.Cu) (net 42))
 (segment (start 73.138 92.929) (end 85.030919 92.929) (width 0.508) (layer F.Cu) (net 42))
 (segment (start 70.231 90.022) (end 71.868 91.659) (width 0.508) (layer F.Cu) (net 42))
 (segment (start 70.231 89.2095) (end 70.231 90.022) (width 0.508) (layer F.Cu) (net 42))
 (segment (start 61.933 99.392) (end 67.888 93.437) (width 0.508) (layer F.Cu) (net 42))
 (segment (start 61.933 100.2045) (end 61.933 99.392) (width 0.508) (layer F.Cu) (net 42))
 (segment (start 67.888 93.437) (end 67.888 93.437) (width 0.508) (layer F.Cu) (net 42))
 (segment (start 67.888 93.437) (end 67.888 93.437) (width 0.508) (layer F.Cu) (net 42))
 (via (at 67.888 93.437) (size 0.8) (drill 0.4) (layers F.Cu B.Cu) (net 42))
 (segment (start 68.287999 93.037001) (end 70.460999 93.037001) (width 0.508) (layer B.Cu) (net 42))
 (segment (start 67.888 93.437) (end 68.287999 93.037001) (width 0.508) (layer B.Cu) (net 42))
 (segment (start 70.460999 93.037001) (end 71.839 91.659) (width 0.508) (layer B.Cu) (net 42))
 (segment (start 71.868 91.659) (end 73.138 92.929) (width 0.508) (layer F.Cu) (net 42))
 (via (at 71.868 91.659) (size 0.8) (drill 0.4) (layers F.Cu B.Cu) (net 42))
 (segment (start 85.030919 95.469) (end 86.233 95.469) (width 0.508) (layer F.Cu) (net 43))
 (segment (start 72.122 95.469) (end 85.030919 95.469) (width 0.508) (layer F.Cu) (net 43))
 (segment (start 66.675 90.022) (end 72.122 95.469) (width 0.508) (layer F.Cu) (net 43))
 (segment (start 66.675 89.2095) (end 66.675 90.022) (width 0.508) (layer F.Cu) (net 43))
 (segment (start 46.736 89.754) (end 50.927 85.563) (width 0.508) (layer F.Cu) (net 17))
 (segment (start 15.621 89.754) (end 46.736 89.754) (width 0.508) (layer F.Cu) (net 17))
 (segment (start 7.62 101.438) (end 7.62 97.755) (width 0.508) (layer F.Cu) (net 17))
 (segment (start 7.62 97.755) (end 15.621 89.754) (width 0.508) (layer F.Cu) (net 17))
 (segment (start 50.927 82.0975) (end 54.991 82.0975) (width 0.508) (layer F.Cu) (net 17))
 (segment (start 52.676 83.912) (end 50.927 83.912) (width 0.508) (layer F.Cu) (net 17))
 (segment (start 54.186 85.422) (end 52.676 83.912) (width 0.508) (layer F.Cu) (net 17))
 (segment (start 54.186 86.2345) (end 54.186 85.422) (width 0.508) (layer F.Cu) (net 17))
 (segment (start 50.927 85.563) (end 50.927 83.912) (width 0.508) (layer F.Cu) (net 17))
 (segment (start 50.927 83.912) (end 50.927 82.0975) (width 0.508) (layer F.Cu) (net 17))
 (segment (start 18.023 69.699) (end 20.865 69.699) (width 0.508) (layer B.Cu) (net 6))
 (segment (start 7.62 83.658) (end 7.62 80.102) (width 0.508) (layer B.Cu) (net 6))
 (segment (start 7.62 80.102) (end 18.023 69.699) (width 0.508) (layer B.Cu) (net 6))
 (segment (start 56.007 103.1795) (end 53.8955 103.1795) (width 0.508) (layer F.Cu) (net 6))
 (segment (start 53.8955 103.1795) (end 46.312 95.596) (width 0.508) (layer F.Cu) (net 6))
 (segment (start 46.312 95.596) (end 25.865 95.596) (width 0.508) (layer F.Cu) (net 6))
 (segment (start 25.865 95.596) (end 25.865 95.596) (width 0.508) (layer F.Cu) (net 6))
 (via (at 25.865 95.596) (size 0.8) (drill 0.4) (layers F.Cu B.Cu) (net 6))
 (segment (start 7.62 87.257) (end 7.62 83.658) (width 0.508) (layer B.Cu) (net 6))
 (segment (start 25.865 95.596) (end 15.959 95.596) (width 0.508) (layer B.Cu) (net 6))
 (segment (start 15.959 95.596) (end 7.62 87.257) (width 0.508) (layer B.Cu) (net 6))
 (segment (start 59.182 79.1225) (end 59.182 68.969) (width 0.508) (layer F.Cu) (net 5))
 (segment (start 59.182 68.969) (end 56.853 66.64) (width 0.508) (layer F.Cu) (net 5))
 (segment (start 56.853 66.64) (end 53.17 66.64) (width 0.508) (layer F.Cu) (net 5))
 (segment (start 53.17 66.64) (end 52.154 67.656) (width 0.508) (layer F.Cu) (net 5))
 (segment (start 52.154 67.656) (end 52.154 71.974) (width 0.508) (layer F.Cu) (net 5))
 (segment (start 52.154 71.974) (end 49.36 74.768) (width 0.508) (layer F.Cu) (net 5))
 (segment (start 49.36 74.768) (end 37.422 74.768) (width 0.508) (layer F.Cu) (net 5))
 (segment (start 35.216 72.562) (end 35.216 69.572) (width 0.508) (layer F.Cu) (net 5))
 (segment (start 37.422 74.768) (end 35.216 72.562) (width 0.508) (layer F.Cu) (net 5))
 (segment (start 63.918 73.6245) (end 63.9175 73.625) (width 0.508) (layer F.Cu) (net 3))
 (segment (start 63.918 69.445) (end 63.918 73.6245) (width 0.508) (layer F.Cu) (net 3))
 (segment (start 63.922 78.7415) (end 61.171 75.9905) (width 0.508) (layer F.Cu) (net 4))
 (segment (start 64.897 78.7415) (end 63.922 78.7415) (width 0.508) (layer F.Cu) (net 4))
 (segment (start 61.171 75.9905) (end 61.171 68.545) (width 0.508) (layer F.Cu) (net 4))
 (segment (start 61.171 68.545) (end 57.615 64.989) (width 0.508) (layer F.Cu) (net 4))
 (segment (start 57.615 64.989) (end 51.519 64.989) (width 0.508) (layer F.Cu) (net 4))
 (segment (start 49.567 66.941) (end 49.567 69.572) (width 0.508) (layer F.Cu) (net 4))
 (segment (start 51.519 64.989) (end 49.567 66.941) (width 0.508) (layer F.Cu) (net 4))
 (segment (start 78.396 75.0215) (end 78.359 75.0585) (width 0.508) (layer F.Cu) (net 1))
 (segment (start 78.396 69.318) (end 78.396 75.0215) (width 0.508) (layer F.Cu) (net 1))
 (segment (start 50.927 79.1225) (end 10.7045 79.1225) (width 0.508) (layer F.Cu) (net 7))
 (segment (start 6.514 74.932) (end 6.514 69.699) (width 0.508) (layer F.Cu) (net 7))
 (segment (start 10.7045 79.1225) (end 6.514 74.932) (width 0.508) (layer F.Cu) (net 7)))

